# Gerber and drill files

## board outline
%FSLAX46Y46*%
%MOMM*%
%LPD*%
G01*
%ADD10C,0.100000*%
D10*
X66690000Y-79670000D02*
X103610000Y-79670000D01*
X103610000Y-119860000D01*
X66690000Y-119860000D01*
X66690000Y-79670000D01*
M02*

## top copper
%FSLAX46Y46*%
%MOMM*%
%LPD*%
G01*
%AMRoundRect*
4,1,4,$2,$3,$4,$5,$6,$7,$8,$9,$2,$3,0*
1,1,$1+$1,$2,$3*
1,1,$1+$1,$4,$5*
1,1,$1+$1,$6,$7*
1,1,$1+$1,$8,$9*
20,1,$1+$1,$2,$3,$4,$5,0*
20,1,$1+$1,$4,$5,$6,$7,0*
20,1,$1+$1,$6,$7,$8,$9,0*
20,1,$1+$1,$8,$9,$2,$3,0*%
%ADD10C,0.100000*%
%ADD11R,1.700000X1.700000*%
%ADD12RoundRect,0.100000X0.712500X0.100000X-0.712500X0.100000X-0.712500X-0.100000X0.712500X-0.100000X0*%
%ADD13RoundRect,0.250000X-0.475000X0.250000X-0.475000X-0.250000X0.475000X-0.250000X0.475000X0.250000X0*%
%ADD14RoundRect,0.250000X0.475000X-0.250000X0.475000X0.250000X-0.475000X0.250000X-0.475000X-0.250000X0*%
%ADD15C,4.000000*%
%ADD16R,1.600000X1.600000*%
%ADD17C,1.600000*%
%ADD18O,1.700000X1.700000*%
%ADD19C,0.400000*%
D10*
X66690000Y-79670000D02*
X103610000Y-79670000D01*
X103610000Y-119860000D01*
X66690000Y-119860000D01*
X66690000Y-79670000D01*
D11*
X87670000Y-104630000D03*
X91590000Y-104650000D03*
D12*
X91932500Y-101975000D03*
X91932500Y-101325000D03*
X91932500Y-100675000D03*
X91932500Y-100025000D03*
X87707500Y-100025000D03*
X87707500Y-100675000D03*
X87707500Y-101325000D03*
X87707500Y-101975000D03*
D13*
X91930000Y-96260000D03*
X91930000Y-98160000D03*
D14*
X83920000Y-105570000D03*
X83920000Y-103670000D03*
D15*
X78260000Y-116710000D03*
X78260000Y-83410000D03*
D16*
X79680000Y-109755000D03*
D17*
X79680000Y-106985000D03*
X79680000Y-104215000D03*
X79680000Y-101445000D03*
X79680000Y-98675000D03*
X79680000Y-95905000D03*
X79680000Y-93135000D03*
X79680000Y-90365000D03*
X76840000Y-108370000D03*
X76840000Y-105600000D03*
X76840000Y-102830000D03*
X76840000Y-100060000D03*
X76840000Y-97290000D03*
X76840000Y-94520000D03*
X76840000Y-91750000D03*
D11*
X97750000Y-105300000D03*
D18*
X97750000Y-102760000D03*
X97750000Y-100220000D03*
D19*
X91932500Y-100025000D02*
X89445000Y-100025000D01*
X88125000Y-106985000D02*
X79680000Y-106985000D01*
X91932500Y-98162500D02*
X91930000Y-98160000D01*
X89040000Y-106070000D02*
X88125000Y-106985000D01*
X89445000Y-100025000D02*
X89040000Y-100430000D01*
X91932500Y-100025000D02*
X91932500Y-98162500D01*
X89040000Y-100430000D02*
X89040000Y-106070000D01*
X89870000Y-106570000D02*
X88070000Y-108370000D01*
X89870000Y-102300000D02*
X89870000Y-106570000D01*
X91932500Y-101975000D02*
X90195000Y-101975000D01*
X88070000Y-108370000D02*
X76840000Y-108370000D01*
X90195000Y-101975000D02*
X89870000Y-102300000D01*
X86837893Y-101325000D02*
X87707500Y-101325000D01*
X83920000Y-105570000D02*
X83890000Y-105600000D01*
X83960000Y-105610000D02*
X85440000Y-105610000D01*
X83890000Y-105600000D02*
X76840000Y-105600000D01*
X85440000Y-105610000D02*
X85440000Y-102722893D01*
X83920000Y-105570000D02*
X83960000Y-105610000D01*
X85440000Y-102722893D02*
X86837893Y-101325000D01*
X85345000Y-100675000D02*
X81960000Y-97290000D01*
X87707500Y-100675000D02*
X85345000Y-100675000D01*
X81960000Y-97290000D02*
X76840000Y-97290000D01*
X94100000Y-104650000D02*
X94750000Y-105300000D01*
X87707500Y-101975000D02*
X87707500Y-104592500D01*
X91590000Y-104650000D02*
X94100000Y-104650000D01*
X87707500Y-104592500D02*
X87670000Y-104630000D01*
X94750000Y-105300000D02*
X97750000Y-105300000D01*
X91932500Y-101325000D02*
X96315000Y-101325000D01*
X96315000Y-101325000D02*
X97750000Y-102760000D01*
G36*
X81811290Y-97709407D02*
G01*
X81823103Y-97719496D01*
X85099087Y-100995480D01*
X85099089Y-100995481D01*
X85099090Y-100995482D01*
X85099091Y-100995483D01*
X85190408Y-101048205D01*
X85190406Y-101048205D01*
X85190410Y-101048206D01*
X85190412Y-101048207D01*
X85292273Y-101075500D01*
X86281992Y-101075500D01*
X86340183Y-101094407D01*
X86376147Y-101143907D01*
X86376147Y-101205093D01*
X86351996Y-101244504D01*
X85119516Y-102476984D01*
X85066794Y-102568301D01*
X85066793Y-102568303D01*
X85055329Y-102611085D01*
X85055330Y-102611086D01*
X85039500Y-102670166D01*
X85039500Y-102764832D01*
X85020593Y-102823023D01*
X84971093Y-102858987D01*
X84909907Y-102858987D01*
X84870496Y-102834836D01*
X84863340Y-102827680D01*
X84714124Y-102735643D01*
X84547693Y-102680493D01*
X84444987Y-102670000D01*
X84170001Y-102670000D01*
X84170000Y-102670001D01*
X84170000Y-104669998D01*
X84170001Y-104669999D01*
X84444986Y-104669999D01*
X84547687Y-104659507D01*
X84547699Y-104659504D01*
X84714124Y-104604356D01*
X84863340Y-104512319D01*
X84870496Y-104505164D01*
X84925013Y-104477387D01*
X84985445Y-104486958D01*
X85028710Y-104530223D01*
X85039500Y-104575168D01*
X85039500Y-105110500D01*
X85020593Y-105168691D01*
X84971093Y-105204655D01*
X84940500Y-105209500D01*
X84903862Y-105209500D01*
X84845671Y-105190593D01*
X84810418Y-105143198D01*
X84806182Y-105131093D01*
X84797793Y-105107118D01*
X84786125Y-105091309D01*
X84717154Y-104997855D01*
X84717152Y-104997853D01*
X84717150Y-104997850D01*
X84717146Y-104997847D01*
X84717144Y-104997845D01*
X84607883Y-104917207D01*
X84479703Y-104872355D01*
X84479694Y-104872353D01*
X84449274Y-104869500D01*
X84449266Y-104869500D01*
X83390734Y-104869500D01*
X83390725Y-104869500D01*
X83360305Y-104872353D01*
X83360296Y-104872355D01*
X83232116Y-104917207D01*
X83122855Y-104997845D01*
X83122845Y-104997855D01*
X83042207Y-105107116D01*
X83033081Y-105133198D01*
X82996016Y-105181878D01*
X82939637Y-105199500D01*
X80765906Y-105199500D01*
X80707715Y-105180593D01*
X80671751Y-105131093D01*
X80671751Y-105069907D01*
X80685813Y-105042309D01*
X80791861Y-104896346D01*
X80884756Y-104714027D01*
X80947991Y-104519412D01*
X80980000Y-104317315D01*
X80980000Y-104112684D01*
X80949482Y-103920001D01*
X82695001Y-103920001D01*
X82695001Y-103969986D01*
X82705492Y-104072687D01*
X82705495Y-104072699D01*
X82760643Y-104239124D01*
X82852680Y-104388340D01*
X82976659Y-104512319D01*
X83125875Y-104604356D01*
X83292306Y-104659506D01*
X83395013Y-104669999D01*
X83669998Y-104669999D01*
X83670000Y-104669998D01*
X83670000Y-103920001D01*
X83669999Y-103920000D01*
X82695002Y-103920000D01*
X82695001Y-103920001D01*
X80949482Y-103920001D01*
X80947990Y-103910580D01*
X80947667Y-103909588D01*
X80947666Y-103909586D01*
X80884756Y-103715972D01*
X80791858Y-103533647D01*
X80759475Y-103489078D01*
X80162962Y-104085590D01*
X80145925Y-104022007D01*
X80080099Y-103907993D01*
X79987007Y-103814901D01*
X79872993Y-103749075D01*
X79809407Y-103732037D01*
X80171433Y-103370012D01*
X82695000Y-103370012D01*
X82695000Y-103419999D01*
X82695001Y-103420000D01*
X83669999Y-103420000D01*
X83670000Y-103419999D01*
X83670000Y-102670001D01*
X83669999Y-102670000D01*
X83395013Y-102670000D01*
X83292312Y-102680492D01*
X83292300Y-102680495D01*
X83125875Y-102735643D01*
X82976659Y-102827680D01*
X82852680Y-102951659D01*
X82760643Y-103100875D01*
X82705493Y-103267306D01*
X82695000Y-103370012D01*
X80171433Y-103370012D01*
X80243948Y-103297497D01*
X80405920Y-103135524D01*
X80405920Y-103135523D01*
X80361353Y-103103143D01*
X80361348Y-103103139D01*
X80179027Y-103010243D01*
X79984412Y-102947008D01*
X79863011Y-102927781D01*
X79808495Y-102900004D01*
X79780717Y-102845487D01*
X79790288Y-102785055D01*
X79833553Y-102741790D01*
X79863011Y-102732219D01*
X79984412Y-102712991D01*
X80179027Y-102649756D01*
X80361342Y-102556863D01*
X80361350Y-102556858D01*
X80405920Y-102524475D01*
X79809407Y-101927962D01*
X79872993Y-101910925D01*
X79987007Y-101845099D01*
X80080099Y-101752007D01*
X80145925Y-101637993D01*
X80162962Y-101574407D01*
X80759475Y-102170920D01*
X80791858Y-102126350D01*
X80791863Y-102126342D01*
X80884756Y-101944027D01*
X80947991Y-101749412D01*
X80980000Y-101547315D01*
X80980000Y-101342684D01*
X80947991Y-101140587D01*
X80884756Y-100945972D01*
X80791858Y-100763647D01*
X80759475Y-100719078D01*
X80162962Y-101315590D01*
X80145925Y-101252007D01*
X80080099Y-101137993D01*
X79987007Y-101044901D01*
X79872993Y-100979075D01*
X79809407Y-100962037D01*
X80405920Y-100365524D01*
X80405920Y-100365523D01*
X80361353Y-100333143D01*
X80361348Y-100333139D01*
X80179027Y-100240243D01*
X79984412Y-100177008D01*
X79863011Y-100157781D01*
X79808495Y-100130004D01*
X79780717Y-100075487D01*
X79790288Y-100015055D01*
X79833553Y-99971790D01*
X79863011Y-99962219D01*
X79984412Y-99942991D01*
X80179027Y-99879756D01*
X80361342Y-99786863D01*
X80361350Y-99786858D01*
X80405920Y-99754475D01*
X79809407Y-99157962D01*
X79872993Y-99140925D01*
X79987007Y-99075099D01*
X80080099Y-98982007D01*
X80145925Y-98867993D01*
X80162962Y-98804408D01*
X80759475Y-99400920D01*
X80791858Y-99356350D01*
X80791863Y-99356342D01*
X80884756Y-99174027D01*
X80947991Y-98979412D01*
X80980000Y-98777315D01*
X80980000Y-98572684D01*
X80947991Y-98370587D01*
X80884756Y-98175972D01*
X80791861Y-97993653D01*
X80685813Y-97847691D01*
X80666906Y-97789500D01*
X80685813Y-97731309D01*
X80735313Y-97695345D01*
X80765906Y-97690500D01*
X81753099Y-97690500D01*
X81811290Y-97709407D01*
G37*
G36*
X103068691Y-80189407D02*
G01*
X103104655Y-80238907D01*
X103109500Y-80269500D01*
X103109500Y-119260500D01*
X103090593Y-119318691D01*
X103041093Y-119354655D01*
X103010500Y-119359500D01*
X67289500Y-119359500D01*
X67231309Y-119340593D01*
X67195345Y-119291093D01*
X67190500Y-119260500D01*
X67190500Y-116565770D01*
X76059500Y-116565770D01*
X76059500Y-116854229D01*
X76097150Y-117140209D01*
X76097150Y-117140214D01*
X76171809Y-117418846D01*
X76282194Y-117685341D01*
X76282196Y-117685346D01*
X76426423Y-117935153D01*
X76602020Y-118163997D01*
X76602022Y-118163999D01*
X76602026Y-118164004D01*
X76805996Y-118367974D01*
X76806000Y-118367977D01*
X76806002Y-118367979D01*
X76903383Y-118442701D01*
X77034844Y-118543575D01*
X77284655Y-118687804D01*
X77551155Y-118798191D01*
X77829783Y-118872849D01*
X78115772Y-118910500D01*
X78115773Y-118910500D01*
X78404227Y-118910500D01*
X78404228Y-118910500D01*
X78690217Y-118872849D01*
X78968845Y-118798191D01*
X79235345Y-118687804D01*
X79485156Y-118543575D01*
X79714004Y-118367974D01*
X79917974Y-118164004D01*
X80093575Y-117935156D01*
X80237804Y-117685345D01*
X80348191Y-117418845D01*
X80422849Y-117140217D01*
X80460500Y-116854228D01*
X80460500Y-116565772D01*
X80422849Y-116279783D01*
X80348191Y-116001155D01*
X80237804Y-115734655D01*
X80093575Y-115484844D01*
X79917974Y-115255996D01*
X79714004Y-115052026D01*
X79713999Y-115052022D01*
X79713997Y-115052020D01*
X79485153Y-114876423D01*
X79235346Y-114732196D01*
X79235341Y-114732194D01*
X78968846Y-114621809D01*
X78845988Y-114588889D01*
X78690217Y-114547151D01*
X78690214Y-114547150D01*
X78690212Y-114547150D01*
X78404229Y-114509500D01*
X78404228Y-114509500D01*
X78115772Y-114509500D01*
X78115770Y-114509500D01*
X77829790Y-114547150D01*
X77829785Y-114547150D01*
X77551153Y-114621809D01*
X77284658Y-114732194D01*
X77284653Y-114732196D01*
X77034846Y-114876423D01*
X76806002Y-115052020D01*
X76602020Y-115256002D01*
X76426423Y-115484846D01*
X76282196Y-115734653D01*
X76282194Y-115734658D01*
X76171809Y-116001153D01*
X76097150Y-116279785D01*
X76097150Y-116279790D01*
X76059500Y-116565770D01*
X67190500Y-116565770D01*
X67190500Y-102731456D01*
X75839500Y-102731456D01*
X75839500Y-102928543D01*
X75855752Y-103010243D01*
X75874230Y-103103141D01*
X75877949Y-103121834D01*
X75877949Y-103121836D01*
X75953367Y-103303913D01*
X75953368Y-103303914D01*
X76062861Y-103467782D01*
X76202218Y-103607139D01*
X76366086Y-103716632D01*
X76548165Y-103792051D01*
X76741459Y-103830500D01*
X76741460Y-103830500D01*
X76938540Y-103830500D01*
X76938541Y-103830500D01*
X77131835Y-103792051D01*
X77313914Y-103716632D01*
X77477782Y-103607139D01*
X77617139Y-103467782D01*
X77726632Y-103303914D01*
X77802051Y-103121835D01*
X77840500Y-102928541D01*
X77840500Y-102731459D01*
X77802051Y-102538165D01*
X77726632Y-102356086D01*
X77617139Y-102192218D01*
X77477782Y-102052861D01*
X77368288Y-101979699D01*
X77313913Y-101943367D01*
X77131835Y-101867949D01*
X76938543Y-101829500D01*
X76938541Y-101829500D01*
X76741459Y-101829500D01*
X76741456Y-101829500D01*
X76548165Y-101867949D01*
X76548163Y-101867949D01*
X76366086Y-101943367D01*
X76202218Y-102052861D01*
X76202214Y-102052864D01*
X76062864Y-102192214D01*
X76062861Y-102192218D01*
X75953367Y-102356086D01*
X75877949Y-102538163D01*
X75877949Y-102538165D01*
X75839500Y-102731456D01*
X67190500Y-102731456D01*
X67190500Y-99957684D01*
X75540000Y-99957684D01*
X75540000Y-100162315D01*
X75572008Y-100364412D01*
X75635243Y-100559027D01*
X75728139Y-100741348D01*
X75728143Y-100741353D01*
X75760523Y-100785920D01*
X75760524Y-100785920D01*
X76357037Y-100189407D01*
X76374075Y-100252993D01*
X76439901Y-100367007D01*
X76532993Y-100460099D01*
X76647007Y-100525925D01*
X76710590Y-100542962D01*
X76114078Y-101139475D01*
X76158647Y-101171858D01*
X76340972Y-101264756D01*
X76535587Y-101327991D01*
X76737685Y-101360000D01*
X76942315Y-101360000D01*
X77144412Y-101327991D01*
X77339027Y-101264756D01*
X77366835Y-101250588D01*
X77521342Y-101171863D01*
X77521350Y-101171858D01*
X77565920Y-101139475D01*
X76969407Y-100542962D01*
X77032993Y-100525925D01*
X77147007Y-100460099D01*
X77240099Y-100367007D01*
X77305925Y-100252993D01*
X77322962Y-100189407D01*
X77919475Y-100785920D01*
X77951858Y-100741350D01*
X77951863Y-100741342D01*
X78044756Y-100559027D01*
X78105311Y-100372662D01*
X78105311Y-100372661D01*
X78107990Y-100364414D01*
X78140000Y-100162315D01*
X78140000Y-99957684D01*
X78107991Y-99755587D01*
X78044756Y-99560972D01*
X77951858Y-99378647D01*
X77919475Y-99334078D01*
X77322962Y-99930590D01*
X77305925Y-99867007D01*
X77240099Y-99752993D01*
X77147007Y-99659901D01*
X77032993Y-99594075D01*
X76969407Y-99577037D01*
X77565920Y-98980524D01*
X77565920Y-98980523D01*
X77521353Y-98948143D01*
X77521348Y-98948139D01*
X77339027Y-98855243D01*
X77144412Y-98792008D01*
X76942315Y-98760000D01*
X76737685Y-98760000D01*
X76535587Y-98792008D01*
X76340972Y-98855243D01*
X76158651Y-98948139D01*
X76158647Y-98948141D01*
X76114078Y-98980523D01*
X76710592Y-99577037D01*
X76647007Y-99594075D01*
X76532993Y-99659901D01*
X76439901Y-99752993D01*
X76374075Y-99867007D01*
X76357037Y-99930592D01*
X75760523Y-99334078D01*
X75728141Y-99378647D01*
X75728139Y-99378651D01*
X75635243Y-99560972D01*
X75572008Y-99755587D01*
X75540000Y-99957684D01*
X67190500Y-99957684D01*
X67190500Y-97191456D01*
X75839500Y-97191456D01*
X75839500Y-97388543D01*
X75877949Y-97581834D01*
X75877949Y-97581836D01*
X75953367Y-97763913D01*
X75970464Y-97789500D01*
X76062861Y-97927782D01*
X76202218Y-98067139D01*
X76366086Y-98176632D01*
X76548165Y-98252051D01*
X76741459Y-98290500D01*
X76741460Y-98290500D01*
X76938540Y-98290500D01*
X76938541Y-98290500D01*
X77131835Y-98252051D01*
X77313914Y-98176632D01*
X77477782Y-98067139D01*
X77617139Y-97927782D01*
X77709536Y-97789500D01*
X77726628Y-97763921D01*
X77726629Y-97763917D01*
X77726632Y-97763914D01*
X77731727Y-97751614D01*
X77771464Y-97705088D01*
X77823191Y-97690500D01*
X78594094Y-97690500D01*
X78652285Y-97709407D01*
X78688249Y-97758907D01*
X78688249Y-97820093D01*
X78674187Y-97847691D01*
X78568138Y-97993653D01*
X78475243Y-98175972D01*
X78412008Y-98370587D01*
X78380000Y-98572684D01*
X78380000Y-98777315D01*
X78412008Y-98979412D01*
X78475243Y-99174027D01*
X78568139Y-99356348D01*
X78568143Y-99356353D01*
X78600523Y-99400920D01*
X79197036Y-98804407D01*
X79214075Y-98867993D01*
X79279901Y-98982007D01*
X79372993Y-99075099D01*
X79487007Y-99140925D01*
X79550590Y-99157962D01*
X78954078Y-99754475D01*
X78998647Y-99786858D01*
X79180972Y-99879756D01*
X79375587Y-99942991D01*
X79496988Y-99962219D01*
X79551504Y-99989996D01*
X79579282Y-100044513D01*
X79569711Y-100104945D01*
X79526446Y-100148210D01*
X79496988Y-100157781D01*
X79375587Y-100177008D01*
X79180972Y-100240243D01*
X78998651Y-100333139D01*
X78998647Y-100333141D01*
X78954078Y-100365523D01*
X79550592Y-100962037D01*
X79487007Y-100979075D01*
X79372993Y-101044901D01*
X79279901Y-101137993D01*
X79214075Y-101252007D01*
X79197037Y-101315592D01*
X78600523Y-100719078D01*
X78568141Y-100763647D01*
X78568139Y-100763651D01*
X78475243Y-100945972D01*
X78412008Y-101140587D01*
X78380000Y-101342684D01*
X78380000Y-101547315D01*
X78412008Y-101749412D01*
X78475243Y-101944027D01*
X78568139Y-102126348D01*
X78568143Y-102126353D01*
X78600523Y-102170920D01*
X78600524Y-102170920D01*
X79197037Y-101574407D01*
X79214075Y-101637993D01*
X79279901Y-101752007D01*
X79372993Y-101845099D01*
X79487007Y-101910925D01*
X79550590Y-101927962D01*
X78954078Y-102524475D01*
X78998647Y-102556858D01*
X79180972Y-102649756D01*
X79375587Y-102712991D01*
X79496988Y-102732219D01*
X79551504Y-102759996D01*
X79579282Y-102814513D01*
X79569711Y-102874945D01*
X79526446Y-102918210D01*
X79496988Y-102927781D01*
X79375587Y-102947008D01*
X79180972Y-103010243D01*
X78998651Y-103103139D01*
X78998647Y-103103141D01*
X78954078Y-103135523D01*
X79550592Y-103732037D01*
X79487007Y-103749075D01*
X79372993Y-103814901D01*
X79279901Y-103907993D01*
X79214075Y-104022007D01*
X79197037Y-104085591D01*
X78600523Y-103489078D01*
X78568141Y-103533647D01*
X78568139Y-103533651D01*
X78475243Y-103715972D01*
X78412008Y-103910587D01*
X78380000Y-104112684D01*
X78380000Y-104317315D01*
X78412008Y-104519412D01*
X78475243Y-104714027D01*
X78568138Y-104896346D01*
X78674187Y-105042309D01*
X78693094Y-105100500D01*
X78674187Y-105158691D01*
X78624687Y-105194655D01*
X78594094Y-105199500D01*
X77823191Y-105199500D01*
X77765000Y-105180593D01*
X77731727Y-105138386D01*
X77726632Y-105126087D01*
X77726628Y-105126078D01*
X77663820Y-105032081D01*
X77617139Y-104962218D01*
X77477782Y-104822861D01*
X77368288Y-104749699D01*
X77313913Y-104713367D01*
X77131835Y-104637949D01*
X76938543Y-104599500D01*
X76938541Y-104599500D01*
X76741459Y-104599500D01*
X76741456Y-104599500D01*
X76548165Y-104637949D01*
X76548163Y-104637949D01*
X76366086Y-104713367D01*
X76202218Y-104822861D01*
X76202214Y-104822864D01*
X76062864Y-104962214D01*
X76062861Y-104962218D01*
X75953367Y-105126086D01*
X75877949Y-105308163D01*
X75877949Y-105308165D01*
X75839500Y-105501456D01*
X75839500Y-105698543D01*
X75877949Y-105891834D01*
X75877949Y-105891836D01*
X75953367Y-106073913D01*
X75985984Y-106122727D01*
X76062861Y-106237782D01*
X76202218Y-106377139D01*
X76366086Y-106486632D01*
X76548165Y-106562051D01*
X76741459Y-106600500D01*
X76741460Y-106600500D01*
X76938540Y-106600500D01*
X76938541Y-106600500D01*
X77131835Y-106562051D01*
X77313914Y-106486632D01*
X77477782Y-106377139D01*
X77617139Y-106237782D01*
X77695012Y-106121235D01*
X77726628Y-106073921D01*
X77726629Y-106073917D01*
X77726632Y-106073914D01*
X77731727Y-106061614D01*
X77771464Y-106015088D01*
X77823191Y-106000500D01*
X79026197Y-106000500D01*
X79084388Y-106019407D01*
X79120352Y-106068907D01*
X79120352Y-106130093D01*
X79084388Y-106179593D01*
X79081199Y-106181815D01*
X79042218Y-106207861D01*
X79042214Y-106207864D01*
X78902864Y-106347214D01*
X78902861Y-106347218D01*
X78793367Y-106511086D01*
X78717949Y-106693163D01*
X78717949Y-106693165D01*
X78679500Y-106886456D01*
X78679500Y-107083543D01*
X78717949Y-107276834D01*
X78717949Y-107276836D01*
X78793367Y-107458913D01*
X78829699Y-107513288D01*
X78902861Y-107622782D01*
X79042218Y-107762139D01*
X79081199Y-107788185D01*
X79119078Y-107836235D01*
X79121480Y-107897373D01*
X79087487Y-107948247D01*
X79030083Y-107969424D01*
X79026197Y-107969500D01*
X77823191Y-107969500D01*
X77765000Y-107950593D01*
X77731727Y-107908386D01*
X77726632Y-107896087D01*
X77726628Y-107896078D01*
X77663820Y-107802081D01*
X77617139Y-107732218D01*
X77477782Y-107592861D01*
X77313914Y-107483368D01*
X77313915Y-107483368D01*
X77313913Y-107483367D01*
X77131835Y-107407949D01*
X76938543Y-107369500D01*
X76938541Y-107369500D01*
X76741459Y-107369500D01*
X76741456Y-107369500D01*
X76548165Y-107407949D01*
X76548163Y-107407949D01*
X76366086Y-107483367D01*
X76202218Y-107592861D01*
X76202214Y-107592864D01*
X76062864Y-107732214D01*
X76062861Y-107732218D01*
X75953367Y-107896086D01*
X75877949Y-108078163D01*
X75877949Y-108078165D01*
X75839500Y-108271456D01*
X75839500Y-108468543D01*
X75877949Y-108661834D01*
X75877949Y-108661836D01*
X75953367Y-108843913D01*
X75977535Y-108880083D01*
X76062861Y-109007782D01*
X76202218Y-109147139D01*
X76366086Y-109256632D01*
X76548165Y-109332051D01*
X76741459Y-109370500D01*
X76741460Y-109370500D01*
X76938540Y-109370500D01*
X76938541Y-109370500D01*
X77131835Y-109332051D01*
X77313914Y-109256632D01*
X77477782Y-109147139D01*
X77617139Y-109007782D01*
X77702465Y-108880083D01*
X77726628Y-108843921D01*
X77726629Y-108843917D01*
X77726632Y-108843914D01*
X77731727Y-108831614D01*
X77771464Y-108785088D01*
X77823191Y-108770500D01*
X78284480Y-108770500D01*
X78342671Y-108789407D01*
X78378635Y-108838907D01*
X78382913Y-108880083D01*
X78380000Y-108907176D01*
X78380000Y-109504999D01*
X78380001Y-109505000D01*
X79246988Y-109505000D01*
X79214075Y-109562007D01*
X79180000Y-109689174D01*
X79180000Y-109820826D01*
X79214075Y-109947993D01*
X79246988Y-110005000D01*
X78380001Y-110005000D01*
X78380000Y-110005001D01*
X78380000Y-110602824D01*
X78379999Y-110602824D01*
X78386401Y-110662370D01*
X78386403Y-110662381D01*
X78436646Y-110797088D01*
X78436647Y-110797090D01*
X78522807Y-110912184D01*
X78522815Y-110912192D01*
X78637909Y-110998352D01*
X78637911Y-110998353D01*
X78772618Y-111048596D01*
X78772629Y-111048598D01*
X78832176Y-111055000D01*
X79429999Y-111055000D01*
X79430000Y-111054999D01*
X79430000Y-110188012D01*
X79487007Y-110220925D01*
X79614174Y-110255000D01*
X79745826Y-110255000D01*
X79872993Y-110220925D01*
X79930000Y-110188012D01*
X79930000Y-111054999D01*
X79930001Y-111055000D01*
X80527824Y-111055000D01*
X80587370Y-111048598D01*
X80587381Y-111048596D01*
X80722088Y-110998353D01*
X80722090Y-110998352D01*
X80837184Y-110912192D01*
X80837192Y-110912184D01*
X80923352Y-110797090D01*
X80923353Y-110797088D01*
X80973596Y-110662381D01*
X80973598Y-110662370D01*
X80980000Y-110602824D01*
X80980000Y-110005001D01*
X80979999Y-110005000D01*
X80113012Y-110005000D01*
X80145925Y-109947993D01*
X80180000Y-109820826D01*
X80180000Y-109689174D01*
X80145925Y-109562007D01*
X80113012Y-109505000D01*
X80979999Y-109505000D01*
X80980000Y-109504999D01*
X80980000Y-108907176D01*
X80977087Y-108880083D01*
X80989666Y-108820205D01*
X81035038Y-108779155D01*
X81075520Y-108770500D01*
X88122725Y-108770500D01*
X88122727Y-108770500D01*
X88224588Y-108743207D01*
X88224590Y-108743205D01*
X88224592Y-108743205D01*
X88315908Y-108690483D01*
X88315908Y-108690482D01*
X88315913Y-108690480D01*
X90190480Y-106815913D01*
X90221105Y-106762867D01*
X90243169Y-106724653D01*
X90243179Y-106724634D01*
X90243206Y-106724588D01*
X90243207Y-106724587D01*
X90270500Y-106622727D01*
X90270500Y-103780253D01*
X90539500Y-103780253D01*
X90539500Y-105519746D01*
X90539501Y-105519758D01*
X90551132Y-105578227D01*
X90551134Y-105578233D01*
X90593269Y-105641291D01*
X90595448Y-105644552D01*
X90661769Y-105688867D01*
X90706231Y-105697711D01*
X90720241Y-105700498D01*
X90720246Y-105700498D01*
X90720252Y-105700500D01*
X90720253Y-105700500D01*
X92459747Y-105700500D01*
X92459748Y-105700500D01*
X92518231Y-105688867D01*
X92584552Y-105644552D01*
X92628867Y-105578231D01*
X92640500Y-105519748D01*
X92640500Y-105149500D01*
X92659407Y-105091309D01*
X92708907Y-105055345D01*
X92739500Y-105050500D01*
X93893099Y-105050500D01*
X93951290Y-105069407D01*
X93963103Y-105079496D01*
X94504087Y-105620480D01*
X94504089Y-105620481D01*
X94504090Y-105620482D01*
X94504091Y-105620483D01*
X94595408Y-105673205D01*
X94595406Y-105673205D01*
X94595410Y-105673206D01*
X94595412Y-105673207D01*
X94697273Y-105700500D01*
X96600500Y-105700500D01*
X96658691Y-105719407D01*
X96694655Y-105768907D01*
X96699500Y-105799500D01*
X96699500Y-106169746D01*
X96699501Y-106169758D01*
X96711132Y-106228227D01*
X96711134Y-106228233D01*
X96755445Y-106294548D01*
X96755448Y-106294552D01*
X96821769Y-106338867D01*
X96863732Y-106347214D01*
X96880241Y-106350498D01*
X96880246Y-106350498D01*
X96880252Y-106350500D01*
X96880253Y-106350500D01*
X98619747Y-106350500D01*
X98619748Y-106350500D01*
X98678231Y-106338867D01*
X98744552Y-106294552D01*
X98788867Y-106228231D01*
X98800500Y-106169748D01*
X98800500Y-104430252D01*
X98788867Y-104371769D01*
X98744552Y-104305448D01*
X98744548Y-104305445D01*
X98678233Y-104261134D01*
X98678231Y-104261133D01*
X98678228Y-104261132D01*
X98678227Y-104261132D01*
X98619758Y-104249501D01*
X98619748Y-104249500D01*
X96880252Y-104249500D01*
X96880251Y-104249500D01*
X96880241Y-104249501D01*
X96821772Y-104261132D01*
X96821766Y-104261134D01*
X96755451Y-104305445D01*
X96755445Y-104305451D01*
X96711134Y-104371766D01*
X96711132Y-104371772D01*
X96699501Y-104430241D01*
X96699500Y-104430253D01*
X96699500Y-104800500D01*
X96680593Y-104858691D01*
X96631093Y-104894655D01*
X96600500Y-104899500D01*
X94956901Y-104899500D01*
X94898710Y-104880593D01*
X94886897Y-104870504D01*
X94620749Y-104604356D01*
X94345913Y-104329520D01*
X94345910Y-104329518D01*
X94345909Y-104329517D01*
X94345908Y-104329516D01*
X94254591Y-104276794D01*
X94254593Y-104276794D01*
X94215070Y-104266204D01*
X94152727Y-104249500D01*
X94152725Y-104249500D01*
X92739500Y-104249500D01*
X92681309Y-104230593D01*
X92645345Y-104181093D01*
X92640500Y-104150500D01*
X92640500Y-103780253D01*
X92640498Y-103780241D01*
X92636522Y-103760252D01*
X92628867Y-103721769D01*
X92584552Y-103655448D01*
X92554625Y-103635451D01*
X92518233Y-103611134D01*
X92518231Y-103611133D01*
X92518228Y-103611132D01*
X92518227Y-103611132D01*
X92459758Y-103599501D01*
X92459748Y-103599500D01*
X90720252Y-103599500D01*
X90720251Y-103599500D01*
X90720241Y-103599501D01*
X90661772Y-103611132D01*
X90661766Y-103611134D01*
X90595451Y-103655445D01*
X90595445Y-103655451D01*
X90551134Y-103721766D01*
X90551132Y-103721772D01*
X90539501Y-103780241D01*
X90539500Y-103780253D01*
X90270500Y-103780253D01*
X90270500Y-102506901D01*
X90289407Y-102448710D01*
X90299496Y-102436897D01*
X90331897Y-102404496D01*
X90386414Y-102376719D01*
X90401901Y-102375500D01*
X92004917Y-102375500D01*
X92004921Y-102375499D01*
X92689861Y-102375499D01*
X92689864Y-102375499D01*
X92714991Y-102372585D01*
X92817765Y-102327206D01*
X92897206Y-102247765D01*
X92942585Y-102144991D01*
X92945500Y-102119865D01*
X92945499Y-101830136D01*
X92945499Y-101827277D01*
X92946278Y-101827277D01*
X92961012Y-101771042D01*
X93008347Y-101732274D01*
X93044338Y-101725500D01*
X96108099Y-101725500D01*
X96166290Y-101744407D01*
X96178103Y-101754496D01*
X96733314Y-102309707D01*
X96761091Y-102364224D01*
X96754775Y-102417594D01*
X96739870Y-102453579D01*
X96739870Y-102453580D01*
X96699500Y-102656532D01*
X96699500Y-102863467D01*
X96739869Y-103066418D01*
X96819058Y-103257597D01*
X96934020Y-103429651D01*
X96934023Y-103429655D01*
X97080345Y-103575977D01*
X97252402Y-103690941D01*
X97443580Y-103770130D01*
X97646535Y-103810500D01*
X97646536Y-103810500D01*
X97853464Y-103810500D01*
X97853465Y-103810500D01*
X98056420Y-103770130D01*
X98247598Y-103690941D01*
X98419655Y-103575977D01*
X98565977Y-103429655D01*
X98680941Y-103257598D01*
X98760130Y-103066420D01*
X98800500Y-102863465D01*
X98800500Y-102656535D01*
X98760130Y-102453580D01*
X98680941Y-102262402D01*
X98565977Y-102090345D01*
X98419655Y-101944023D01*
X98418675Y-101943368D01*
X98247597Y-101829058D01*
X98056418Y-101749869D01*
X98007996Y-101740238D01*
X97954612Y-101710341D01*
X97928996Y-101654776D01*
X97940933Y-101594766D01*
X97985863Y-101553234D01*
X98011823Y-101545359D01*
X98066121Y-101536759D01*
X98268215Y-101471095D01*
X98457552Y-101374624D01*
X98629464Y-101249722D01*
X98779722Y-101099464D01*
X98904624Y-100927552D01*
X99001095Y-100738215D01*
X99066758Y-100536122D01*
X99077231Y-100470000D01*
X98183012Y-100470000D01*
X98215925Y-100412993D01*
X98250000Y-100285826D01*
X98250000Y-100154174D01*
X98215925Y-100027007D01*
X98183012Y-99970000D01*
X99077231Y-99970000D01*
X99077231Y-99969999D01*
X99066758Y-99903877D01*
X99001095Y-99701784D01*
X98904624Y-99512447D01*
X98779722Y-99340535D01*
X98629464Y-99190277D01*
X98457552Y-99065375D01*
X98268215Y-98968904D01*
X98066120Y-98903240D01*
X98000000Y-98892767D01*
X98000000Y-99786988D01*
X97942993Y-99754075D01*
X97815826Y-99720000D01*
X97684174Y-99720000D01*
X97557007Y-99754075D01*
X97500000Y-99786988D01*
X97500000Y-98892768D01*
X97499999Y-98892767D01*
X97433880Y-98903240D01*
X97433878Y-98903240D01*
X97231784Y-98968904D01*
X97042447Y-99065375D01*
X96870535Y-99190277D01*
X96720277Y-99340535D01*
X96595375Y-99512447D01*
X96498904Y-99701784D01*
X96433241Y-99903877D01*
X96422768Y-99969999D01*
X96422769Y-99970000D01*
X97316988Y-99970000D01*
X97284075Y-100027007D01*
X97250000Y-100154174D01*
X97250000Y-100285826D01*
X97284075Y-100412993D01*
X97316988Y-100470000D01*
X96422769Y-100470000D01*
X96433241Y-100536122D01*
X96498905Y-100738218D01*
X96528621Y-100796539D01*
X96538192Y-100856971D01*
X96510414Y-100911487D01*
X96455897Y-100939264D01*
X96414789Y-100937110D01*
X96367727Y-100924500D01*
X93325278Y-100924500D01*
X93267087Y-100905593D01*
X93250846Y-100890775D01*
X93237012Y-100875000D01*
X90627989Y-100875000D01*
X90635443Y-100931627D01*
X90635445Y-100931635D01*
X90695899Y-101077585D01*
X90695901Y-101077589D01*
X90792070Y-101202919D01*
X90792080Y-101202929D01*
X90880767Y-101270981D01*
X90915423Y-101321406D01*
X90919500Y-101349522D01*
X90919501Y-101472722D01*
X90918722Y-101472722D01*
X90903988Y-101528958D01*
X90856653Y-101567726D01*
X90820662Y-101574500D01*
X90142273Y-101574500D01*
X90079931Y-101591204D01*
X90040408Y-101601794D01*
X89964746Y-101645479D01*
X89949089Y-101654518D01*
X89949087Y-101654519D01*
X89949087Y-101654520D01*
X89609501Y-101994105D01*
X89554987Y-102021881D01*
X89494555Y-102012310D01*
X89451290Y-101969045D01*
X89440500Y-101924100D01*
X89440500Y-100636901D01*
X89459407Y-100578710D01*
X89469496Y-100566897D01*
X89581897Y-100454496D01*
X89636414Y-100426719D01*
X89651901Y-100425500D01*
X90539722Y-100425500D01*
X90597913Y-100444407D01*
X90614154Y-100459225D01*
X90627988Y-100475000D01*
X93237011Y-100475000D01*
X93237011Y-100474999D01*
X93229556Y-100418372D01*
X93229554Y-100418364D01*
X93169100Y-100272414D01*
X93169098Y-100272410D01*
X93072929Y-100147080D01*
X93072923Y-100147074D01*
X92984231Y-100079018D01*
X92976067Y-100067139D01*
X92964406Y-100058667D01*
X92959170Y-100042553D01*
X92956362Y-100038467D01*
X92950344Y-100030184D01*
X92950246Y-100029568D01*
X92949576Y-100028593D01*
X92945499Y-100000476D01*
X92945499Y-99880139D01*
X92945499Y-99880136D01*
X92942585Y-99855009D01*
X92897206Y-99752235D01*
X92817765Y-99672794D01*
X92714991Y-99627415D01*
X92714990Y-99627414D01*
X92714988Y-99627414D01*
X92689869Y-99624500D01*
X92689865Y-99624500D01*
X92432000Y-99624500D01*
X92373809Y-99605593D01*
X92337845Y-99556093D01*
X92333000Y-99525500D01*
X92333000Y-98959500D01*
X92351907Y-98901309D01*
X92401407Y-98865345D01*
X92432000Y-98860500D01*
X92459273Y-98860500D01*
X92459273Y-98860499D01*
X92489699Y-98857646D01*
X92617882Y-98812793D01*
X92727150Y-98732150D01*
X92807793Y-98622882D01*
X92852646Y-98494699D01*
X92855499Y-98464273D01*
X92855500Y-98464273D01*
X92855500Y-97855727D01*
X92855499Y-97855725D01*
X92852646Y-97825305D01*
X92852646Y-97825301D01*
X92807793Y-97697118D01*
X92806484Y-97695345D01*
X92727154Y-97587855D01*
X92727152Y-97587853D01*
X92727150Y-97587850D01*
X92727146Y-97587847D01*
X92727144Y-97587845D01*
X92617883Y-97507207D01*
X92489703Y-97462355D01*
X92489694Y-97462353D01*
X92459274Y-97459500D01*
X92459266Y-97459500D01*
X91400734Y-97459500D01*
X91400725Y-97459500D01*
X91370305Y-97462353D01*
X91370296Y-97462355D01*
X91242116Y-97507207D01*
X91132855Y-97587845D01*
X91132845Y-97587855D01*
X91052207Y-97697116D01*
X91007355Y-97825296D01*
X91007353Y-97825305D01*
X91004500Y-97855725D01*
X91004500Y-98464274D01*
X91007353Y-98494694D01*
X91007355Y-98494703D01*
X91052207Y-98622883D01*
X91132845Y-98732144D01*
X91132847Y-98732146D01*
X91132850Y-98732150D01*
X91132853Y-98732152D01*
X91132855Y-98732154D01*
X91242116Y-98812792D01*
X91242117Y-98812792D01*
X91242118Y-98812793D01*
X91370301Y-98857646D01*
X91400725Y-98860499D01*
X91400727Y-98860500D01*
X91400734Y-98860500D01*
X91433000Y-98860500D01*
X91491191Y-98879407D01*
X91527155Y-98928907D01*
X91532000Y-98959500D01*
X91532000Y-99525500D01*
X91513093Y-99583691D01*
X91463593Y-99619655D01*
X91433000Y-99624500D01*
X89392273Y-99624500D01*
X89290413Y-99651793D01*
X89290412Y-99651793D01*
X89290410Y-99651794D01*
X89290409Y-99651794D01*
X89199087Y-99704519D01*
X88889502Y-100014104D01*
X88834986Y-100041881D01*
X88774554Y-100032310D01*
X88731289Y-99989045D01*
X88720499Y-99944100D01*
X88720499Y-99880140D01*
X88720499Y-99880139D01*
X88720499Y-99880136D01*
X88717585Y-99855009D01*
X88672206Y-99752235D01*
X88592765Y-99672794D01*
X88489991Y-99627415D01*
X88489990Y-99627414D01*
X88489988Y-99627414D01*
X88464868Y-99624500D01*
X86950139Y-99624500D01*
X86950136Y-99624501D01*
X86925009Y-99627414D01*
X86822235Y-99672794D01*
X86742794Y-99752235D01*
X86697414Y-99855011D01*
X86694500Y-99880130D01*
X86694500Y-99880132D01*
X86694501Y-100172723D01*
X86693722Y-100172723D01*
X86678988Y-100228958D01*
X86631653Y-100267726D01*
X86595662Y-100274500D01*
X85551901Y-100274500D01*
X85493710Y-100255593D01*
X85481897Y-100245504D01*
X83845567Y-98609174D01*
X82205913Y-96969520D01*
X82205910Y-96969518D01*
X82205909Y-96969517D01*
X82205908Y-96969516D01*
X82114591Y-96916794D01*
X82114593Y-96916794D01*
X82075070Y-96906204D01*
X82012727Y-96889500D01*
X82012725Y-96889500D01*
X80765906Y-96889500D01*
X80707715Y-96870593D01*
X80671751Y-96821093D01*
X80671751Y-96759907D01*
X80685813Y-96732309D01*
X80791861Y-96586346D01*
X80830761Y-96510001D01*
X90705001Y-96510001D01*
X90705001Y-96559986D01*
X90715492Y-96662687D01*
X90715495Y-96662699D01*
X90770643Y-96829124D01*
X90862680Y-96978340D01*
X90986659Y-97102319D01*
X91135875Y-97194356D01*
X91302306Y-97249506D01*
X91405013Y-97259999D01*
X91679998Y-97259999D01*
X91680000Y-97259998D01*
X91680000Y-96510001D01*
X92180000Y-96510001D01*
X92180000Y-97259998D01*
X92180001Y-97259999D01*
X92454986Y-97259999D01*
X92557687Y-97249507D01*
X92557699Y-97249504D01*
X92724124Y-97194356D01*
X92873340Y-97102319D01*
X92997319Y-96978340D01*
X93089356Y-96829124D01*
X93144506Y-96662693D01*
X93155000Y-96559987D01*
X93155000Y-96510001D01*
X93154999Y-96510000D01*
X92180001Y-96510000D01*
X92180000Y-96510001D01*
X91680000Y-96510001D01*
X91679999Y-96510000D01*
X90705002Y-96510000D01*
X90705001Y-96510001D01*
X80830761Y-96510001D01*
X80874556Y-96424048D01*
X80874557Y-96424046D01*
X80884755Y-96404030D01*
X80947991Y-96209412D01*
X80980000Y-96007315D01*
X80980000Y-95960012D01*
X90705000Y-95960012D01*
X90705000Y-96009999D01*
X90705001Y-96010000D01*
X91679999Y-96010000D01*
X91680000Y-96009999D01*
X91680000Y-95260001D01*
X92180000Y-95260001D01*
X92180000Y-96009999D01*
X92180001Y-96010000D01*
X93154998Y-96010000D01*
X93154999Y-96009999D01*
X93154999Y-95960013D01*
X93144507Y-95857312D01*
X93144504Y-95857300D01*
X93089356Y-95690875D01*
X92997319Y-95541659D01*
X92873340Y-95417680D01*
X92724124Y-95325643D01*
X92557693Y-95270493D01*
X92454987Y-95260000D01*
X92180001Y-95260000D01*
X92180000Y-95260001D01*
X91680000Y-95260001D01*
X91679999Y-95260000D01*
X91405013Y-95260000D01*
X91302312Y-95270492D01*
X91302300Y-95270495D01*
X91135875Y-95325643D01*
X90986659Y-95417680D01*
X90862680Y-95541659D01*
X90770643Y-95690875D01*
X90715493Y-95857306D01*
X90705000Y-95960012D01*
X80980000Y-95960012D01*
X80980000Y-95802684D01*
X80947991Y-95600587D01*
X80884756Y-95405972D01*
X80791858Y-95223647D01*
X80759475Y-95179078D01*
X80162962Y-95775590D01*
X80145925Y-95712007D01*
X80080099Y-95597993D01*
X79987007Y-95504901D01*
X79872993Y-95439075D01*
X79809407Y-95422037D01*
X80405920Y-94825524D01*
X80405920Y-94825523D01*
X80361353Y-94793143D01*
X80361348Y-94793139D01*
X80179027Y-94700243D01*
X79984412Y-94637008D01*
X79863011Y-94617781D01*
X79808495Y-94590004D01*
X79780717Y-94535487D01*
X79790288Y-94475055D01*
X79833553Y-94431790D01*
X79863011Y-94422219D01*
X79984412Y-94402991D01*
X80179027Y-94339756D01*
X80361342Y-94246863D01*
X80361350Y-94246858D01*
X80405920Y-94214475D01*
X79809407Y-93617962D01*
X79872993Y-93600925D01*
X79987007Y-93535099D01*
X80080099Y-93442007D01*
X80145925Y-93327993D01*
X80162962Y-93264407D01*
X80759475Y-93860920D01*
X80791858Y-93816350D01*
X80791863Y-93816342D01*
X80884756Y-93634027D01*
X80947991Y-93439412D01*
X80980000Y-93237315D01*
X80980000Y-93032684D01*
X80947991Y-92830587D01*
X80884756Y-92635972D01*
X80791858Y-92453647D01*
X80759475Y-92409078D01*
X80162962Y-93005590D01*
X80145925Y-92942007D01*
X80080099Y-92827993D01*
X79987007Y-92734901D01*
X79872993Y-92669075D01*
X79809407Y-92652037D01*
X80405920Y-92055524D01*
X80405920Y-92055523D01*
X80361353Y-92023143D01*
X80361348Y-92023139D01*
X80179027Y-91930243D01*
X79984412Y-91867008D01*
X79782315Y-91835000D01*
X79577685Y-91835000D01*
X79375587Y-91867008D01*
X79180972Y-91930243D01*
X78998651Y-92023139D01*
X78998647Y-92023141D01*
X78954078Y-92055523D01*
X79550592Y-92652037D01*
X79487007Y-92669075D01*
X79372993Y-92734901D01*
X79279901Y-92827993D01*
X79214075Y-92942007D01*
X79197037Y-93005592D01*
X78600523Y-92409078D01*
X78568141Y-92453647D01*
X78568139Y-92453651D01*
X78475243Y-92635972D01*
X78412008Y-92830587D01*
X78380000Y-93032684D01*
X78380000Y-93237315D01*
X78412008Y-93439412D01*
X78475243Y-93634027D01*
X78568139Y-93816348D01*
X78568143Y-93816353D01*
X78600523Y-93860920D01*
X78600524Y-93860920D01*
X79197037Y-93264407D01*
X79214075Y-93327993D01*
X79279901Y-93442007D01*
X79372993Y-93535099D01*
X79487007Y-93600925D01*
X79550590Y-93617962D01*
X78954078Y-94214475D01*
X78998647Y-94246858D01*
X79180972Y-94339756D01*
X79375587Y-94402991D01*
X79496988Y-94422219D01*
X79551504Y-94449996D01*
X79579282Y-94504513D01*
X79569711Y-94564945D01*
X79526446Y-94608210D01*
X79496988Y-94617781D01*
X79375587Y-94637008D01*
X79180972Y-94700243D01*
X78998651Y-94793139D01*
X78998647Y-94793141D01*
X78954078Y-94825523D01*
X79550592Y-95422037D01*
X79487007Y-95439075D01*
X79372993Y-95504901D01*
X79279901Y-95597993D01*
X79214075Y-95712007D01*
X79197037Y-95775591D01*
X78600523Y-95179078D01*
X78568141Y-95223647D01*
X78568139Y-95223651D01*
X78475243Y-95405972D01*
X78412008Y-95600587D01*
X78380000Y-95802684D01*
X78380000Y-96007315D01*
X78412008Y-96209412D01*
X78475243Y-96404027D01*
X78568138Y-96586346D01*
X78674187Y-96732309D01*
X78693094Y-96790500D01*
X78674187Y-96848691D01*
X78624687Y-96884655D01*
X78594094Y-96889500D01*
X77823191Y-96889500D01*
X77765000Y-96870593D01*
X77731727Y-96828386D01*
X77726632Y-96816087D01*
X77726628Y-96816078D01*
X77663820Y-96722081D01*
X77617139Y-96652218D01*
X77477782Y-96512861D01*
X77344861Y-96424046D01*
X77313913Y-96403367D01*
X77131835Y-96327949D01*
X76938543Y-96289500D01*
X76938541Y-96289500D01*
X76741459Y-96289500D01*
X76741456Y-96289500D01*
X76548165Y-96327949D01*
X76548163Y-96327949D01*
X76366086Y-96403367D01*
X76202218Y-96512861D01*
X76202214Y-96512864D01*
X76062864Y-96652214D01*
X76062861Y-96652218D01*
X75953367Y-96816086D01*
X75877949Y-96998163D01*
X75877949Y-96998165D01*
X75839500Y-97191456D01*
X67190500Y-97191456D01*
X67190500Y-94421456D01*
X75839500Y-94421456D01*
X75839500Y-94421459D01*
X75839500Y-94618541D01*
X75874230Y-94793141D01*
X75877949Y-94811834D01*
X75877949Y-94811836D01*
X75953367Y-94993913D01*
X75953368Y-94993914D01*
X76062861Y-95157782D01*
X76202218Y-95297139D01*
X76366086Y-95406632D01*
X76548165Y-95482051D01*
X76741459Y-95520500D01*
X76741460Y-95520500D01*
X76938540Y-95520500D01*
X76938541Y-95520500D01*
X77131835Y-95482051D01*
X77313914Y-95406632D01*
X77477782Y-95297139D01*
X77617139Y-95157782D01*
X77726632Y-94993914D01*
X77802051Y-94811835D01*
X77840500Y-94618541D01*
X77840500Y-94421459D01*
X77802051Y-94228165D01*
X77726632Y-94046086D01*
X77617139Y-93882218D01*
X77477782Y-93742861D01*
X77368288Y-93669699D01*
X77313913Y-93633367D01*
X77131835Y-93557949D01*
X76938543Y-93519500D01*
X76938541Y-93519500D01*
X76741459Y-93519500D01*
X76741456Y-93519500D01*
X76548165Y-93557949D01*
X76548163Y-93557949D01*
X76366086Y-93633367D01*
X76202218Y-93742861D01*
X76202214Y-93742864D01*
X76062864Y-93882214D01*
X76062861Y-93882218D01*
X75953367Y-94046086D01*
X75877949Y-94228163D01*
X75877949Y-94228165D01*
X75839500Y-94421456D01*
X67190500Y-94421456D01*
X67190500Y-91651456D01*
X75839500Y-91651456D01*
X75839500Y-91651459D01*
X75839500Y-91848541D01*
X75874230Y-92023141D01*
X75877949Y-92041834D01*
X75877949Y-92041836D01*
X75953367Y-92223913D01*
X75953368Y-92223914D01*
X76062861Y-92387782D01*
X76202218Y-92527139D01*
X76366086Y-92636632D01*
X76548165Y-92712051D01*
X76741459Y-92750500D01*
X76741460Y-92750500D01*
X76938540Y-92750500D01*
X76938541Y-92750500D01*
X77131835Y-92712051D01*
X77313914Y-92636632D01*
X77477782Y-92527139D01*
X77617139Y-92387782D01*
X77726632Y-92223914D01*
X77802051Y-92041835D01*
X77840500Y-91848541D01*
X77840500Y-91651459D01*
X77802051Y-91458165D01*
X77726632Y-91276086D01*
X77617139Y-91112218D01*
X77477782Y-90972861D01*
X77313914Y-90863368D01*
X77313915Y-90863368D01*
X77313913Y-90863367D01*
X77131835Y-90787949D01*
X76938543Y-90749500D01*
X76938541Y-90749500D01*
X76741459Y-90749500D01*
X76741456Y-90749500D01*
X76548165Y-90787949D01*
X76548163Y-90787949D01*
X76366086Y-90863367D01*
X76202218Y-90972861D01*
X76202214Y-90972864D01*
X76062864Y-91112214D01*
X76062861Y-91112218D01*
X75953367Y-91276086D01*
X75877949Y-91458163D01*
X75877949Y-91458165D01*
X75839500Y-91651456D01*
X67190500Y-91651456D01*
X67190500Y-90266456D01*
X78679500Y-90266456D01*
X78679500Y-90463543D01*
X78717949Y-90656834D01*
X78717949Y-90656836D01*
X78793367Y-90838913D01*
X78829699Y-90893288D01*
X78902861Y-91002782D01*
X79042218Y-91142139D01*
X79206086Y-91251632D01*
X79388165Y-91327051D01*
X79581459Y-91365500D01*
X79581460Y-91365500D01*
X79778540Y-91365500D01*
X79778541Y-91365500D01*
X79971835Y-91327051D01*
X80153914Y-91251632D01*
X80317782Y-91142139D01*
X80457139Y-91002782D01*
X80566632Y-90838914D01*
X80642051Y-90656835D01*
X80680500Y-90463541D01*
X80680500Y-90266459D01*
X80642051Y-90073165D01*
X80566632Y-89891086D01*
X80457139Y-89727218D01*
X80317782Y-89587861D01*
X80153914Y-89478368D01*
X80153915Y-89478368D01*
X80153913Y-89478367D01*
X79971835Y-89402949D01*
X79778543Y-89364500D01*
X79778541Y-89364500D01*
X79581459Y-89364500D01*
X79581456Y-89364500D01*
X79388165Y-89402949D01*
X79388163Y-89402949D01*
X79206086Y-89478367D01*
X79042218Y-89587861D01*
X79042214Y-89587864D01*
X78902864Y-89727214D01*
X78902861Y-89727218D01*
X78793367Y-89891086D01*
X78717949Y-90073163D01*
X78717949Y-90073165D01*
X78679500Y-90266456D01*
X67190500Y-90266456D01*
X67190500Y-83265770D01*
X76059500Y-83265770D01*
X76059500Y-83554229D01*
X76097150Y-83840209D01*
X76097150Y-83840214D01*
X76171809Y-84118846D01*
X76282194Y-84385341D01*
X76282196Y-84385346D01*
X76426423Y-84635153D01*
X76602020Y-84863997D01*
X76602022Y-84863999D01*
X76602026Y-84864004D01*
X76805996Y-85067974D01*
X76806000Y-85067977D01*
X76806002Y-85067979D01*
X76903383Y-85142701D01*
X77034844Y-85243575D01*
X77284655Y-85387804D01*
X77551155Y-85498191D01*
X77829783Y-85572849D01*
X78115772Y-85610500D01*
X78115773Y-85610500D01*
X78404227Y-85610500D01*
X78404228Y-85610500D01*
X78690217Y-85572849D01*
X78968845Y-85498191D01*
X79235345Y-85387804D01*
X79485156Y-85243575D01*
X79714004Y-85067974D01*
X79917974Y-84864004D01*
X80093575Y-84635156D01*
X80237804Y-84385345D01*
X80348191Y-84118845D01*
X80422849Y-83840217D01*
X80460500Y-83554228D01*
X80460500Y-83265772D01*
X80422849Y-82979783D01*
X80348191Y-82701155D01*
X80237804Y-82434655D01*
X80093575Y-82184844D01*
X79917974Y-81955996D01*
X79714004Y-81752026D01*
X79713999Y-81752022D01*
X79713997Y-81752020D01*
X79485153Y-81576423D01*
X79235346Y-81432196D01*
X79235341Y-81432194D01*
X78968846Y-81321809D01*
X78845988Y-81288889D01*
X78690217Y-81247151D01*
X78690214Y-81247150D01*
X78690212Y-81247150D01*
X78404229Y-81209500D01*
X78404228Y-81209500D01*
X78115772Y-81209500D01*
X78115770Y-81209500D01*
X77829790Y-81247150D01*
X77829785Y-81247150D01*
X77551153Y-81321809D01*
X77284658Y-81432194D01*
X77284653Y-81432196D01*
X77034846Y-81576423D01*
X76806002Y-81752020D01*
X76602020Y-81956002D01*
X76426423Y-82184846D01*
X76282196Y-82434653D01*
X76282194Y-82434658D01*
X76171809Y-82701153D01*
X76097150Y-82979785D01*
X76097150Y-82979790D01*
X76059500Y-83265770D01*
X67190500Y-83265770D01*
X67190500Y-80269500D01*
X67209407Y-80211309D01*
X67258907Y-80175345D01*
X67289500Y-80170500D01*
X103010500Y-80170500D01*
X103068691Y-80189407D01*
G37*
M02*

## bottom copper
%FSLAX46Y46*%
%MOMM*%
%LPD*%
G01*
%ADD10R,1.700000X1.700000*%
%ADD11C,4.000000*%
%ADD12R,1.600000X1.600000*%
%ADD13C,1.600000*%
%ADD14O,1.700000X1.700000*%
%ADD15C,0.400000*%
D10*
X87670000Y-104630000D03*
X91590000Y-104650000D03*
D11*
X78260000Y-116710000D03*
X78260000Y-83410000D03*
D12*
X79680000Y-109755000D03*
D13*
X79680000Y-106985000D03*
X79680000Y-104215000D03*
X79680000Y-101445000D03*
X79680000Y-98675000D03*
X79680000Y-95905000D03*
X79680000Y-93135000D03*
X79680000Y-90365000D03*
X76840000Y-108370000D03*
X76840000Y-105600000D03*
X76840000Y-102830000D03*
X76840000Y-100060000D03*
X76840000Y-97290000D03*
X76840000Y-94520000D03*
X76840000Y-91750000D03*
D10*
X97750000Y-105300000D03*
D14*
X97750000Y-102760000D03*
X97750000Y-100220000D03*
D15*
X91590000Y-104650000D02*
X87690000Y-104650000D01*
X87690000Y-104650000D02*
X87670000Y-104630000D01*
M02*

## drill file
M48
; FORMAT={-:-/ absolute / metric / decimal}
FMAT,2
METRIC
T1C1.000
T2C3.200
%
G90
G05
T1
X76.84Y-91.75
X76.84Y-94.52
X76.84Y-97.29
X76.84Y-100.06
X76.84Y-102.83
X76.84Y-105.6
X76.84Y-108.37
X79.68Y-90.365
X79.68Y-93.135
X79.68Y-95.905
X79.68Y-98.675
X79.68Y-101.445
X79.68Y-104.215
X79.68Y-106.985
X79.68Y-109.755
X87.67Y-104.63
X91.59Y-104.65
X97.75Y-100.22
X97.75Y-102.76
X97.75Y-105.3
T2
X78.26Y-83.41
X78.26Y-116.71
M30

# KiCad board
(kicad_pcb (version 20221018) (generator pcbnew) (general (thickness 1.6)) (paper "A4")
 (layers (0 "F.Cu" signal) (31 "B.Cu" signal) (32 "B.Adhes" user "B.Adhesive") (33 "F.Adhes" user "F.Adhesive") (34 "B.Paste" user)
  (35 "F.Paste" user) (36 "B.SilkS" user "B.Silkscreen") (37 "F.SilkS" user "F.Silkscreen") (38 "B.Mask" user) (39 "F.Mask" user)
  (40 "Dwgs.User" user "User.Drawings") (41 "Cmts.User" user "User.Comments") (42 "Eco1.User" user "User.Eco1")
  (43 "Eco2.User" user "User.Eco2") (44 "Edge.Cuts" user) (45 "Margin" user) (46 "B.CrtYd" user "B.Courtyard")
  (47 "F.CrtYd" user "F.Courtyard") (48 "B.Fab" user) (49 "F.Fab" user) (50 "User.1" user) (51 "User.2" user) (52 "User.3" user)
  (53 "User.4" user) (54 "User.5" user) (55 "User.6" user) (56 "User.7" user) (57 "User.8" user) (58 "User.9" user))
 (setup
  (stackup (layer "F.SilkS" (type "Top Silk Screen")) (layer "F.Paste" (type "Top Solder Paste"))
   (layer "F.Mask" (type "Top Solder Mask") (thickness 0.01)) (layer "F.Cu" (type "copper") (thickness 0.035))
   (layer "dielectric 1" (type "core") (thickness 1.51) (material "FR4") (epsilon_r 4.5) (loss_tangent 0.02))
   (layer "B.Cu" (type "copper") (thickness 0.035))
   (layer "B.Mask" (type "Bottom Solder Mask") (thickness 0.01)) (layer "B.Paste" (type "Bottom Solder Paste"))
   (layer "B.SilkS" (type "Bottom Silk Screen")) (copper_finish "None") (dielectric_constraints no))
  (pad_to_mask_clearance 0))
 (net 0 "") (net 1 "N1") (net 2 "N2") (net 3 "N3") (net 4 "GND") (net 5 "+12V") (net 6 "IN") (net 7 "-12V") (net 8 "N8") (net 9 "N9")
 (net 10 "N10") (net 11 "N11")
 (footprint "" (layer "F.Cu") (at 87.67 104.63)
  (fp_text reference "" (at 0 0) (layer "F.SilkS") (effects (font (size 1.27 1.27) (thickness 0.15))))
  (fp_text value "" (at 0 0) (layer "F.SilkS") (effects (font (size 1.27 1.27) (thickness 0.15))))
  (pad "1" thru_hole rect (at 0 0) (size 1.7 1.7) (drill 1) (layers "*.Cu" "*.Mask") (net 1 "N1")))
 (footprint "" (layer "F.Cu") (at 91.59 104.65)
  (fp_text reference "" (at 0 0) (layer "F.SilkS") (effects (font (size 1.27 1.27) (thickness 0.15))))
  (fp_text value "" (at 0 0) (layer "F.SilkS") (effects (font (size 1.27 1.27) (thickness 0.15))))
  (pad "1" thru_hole rect (at 0 0) (size 1.7 1.7) (drill 1) (layers "*.Cu" "*.Mask") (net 1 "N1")))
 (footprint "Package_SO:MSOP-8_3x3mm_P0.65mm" (layer "F.Cu") (at 89.82 101 180)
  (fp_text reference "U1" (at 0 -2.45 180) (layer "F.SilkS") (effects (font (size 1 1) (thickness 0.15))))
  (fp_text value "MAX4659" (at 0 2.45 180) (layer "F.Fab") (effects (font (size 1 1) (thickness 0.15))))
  (pad "1" smd roundrect (at -2.1125 -0.975 180) (size 1.625 0.4) (layers "F.Cu" "F.Paste" "F.Mask") (roundrect_rratio 0.25) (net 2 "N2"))
  (pad "2" smd roundrect (at -2.1125 -0.325 180) (size 1.625 0.4) (layers "F.Cu" "F.Paste" "F.Mask") (roundrect_rratio 0.25) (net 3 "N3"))
  (pad "3" smd roundrect (at -2.1125 0.325 180) (size 1.625 0.4) (layers "F.Cu" "F.Paste" "F.Mask") (roundrect_rratio 0.25) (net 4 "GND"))
  (pad "4" smd roundrect (at -2.1125 0.975 180) (size 1.625 0.4) (layers "F.Cu" "F.Paste" "F.Mask") (roundrect_rratio 0.25) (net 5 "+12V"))
  (pad "5" smd roundrect (at 2.1125 0.975 180) (size 1.625 0.4) (layers "F.Cu" "F.Paste" "F.Mask") (roundrect_rratio 0.25))
  (pad "6" smd roundrect (at 2.1125 0.325 180) (size 1.625 0.4) (layers "F.Cu" "F.Paste" "F.Mask") (roundrect_rratio 0.25) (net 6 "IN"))
  (pad "7" smd roundrect (at 2.1125 -0.325 180) (size 1.625 0.4) (layers "F.Cu" "F.Paste" "F.Mask") (roundrect_rratio 0.25) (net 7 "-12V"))
  (pad "8" smd roundrect (at 2.1125 -0.975 180) (size 1.625 0.4) (layers "F.Cu" "F.Paste" "F.Mask") (roundrect_rratio 0.25) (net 1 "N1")))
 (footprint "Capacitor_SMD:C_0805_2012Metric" (layer "F.Cu") (at 91.93 97.21 -90)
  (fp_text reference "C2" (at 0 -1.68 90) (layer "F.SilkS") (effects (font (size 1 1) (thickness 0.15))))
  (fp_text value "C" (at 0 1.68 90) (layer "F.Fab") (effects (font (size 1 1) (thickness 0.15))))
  (pad "1" smd roundrect (at -0.95 0 270) (size 1 1.45) (layers "F.Cu" "F.Paste" "F.Mask") (roundrect_rratio 0.25) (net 4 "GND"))
  (pad "2" smd roundrect (at 0.95 0 270) (size 1 1.45) (layers "F.Cu" "F.Paste" "F.Mask") (roundrect_rratio 0.25) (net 5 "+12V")))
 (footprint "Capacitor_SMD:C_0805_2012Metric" (layer "F.Cu") (at 83.92 104.62 90)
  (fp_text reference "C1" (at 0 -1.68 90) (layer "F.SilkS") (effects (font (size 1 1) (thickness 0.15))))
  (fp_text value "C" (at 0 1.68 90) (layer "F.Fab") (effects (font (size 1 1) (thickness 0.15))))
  (pad "1" smd roundrect (at -0.95 0 90) (size 1 1.45) (layers "F.Cu" "F.Paste" "F.Mask") (roundrect_rratio 0.25) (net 7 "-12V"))
  (pad "2" smd roundrect (at 0.95 0 90) (size 1 1.45) (layers "F.Cu" "F.Paste" "F.Mask") (roundrect_rratio 0.25) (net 4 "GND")))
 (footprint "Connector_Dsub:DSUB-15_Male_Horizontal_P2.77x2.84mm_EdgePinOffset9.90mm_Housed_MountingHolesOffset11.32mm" (layer "B.Cu")
  (at 79.68 109.755 90)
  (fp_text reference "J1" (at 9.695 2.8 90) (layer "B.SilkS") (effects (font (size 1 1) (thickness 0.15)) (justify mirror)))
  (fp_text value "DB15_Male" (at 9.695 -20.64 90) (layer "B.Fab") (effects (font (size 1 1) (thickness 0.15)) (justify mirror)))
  (pad "0" thru_hole circle (at -6.955 -1.42 90) (size 4 4) (drill 3.2) (layers "*.Cu" "*.Mask"))
  (pad "0" thru_hole circle (at 26.345 -1.42 90) (size 4 4) (drill 3.2) (layers "*.Cu" "*.Mask"))
  (pad "1" thru_hole rect (at 0 0 90) (size 1.6 1.6) (drill 1) (layers "*.Cu" "*.Mask") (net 4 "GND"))
  (pad "2" thru_hole circle (at 2.77 0 90) (size 1.6 1.6) (drill 1) (layers "*.Cu" "*.Mask") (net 5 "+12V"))
  (pad "3" thru_hole circle (at 5.54 0 90) (size 1.6 1.6) (drill 1) (layers "*.Cu" "*.Mask") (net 4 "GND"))
  (pad "4" thru_hole circle (at 8.31 0 90) (size 1.6 1.6) (drill 1) (layers "*.Cu" "*.Mask") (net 4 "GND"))
  (pad "5" thru_hole circle (at 11.08 0 90) (size 1.6 1.6) (drill 1) (layers "*.Cu" "*.Mask") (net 4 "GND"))
  (pad "6" thru_hole circle (at 13.85 0 90) (size 1.6 1.6) (drill 1) (layers "*.Cu" "*.Mask") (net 4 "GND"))
  (pad "7" thru_hole circle (at 16.62 0 90) (size 1.6 1.6) (drill 1) (layers "*.Cu" "*.Mask") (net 4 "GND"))
  (pad "8" thru_hole circle (at 19.39 0 90) (size 1.6 1.6) (drill 1) (layers "*.Cu" "*.Mask") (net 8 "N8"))
  (pad "9" thru_hole circle (at 1.385 -2.84 90) (size 1.6 1.6) (drill 1) (layers "*.Cu" "*.Mask") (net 2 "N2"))
  (pad "10" thru_hole circle (at 4.155 -2.84 90) (size 1.6 1.6) (drill 1) (layers "*.Cu" "*.Mask") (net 7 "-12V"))
  (pad "11" thru_hole circle (at 6.925 -2.84 90) (size 1.6 1.6) (drill 1) (layers "*.Cu" "*.Mask") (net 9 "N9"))
  (pad "12" thru_hole circle (at 9.695 -2.84 90) (size 1.6 1.6) (drill 1) (layers "*.Cu" "*.Mask") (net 4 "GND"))
  (pad "13" thru_hole circle (at 12.465 -2.84 90) (size 1.6 1.6) (drill 1) (layers "*.Cu" "*.Mask") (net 6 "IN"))
  (pad "14" thru_hole circle (at 15.235 -2.84 90) (size 1.6 1.6) (drill 1) (layers "*.Cu" "*.Mask") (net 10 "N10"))
  (pad "15" thru_hole circle (at 18.005 -2.84 90) (size 1.6 1.6) (drill 1) (layers "*.Cu" "*.Mask") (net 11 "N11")))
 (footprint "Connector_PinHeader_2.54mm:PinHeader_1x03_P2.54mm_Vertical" (layer "B.Cu") (at 97.75 105.3)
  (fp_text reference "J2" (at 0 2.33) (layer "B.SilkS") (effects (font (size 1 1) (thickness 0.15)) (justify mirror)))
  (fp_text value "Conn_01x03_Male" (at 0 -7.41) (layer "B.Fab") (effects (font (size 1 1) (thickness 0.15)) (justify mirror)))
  (pad "1" thru_hole rect (at 0 0) (size 1.7 1.7) (drill 1) (layers "*.Cu" "*.Mask") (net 1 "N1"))
  (pad "2" thru_hole oval (at 0 -2.54) (size 1.7 1.7) (drill 1) (layers "*.Cu" "*.Mask") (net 3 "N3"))
  (pad "3" thru_hole oval (at 0 -5.08) (size 1.7 1.7) (drill 1) (layers "*.Cu" "*.Mask") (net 4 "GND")))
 (gr_rect (start 66.69 79.67) (end 103.61 119.86) (stroke (width 0.1) (type default)) (fill none) (layer "F.Cu"))
 (gr_rect (start 66.69 79.67) (end 103.61 119.86) (stroke (width 0.1) (type default)) (fill none) (layer "Edge.Cuts"))
 (segment (start 91.9325 100.025) (end 89.445 100.025) (width 0.4) (layer "F.Cu") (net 5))
 (segment (start 88.125 106.985) (end 79.68 106.985) (width 0.4) (layer "F.Cu") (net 5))
 (segment (start 91.9325 98.1625) (end 91.93 98.16) (width 0.4) (layer "F.Cu") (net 5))
 (segment (start 89.04 106.07) (end 88.125 106.985) (width 0.4) (layer "F.Cu") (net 5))
 (segment (start 89.445 100.025) (end 89.04 100.43) (width 0.4) (layer "F.Cu") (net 5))
 (segment (start 91.9325 100.025) (end 91.9325 98.1625) (width 0.4) (layer "F.Cu") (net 5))
 (segment (start 89.04 100.43) (end 89.04 106.07) (width 0.4) (layer "F.Cu") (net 5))
 (segment (start 89.87 106.57) (end 88.07 108.37) (width 0.4) (layer "F.Cu") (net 2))
 (segment (start 89.87 102.3) (end 89.87 106.57) (width 0.4) (layer "F.Cu") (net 2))
 (segment (start 91.9325 101.975) (end 90.195 101.975) (width 0.4) (layer "F.Cu") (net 2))
 (segment (start 88.07 108.37) (end 76.84 108.37) (width 0.4) (layer "F.Cu") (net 2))
 (segment (start 90.195 101.975) (end 89.87 102.3) (width 0.4) (layer "F.Cu") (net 2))
 (segment (start 86.837893 101.325) (end 87.7075 101.325) (width 0.4) (layer "F.Cu") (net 7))
 (segment (start 83.92 105.57) (end 83.89 105.6) (width 0.4) (layer "F.Cu") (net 7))
 (segment (start 83.96 105.61) (end 85.44 105.61) (width 0.4) (layer "F.Cu") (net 7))
 (segment (start 83.89 105.6) (end 76.84 105.6) (width 0.4) (layer "F.Cu") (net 7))
 (segment (start 85.44 105.61) (end 85.44 102.722893) (width 0.4) (layer "F.Cu") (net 7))
 (segment (start 83.92 105.57) (end 83.96 105.61) (width 0.4) (layer "F.Cu") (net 7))
 (segment (start 85.44 102.722893) (end 86.837893 101.325) (width 0.4) (layer "F.Cu") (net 7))
 (segment (start 85.345 100.675) (end 81.96 97.29) (width 0.4) (layer "F.Cu") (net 6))
 (segment (start 87.7075 100.675) (end 85.345 100.675) (width 0.4) (layer "F.Cu") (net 6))
 (segment (start 81.96 97.29) (end 76.84 97.29) (width 0.4) (layer "F.Cu") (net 6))
 (segment (start 94.1 104.65) (end 94.75 105.3) (width 0.4) (layer "F.Cu") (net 1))
 (segment (start 87.7075 101.975) (end 87.7075 104.5925) (width 0.4) (layer "F.Cu") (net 1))
 (segment (start 91.59 104.65) (end 94.1 104.65) (width 0.4) (layer "F.Cu") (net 1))
 (segment (start 87.7075 104.5925) (end 87.67 104.63) (width 0.4) (layer "F.Cu") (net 1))
 (segment (start 94.75 105.3) (end 97.75 105.3) (width 0.4) (layer "F.Cu") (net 1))
 (segment (start 91.59 104.65) (end 87.69 104.65) (width 0.4) (layer "B.Cu") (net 1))
 (segment (start 87.69 104.65) (end 87.67 104.63) (width 0.4) (layer "B.Cu") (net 1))
 (segment (start 91.9325 101.325) (end 96.315 101.325) (width 0.4) (layer "F.Cu") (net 3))
 (segment (start 96.315 101.325) (end 97.75 102.76) (width 0.4) (layer "F.Cu") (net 3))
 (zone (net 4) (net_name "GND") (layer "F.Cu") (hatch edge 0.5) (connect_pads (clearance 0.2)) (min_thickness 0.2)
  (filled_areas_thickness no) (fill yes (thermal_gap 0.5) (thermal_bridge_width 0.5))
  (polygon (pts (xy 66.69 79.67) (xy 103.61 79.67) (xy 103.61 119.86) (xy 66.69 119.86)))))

